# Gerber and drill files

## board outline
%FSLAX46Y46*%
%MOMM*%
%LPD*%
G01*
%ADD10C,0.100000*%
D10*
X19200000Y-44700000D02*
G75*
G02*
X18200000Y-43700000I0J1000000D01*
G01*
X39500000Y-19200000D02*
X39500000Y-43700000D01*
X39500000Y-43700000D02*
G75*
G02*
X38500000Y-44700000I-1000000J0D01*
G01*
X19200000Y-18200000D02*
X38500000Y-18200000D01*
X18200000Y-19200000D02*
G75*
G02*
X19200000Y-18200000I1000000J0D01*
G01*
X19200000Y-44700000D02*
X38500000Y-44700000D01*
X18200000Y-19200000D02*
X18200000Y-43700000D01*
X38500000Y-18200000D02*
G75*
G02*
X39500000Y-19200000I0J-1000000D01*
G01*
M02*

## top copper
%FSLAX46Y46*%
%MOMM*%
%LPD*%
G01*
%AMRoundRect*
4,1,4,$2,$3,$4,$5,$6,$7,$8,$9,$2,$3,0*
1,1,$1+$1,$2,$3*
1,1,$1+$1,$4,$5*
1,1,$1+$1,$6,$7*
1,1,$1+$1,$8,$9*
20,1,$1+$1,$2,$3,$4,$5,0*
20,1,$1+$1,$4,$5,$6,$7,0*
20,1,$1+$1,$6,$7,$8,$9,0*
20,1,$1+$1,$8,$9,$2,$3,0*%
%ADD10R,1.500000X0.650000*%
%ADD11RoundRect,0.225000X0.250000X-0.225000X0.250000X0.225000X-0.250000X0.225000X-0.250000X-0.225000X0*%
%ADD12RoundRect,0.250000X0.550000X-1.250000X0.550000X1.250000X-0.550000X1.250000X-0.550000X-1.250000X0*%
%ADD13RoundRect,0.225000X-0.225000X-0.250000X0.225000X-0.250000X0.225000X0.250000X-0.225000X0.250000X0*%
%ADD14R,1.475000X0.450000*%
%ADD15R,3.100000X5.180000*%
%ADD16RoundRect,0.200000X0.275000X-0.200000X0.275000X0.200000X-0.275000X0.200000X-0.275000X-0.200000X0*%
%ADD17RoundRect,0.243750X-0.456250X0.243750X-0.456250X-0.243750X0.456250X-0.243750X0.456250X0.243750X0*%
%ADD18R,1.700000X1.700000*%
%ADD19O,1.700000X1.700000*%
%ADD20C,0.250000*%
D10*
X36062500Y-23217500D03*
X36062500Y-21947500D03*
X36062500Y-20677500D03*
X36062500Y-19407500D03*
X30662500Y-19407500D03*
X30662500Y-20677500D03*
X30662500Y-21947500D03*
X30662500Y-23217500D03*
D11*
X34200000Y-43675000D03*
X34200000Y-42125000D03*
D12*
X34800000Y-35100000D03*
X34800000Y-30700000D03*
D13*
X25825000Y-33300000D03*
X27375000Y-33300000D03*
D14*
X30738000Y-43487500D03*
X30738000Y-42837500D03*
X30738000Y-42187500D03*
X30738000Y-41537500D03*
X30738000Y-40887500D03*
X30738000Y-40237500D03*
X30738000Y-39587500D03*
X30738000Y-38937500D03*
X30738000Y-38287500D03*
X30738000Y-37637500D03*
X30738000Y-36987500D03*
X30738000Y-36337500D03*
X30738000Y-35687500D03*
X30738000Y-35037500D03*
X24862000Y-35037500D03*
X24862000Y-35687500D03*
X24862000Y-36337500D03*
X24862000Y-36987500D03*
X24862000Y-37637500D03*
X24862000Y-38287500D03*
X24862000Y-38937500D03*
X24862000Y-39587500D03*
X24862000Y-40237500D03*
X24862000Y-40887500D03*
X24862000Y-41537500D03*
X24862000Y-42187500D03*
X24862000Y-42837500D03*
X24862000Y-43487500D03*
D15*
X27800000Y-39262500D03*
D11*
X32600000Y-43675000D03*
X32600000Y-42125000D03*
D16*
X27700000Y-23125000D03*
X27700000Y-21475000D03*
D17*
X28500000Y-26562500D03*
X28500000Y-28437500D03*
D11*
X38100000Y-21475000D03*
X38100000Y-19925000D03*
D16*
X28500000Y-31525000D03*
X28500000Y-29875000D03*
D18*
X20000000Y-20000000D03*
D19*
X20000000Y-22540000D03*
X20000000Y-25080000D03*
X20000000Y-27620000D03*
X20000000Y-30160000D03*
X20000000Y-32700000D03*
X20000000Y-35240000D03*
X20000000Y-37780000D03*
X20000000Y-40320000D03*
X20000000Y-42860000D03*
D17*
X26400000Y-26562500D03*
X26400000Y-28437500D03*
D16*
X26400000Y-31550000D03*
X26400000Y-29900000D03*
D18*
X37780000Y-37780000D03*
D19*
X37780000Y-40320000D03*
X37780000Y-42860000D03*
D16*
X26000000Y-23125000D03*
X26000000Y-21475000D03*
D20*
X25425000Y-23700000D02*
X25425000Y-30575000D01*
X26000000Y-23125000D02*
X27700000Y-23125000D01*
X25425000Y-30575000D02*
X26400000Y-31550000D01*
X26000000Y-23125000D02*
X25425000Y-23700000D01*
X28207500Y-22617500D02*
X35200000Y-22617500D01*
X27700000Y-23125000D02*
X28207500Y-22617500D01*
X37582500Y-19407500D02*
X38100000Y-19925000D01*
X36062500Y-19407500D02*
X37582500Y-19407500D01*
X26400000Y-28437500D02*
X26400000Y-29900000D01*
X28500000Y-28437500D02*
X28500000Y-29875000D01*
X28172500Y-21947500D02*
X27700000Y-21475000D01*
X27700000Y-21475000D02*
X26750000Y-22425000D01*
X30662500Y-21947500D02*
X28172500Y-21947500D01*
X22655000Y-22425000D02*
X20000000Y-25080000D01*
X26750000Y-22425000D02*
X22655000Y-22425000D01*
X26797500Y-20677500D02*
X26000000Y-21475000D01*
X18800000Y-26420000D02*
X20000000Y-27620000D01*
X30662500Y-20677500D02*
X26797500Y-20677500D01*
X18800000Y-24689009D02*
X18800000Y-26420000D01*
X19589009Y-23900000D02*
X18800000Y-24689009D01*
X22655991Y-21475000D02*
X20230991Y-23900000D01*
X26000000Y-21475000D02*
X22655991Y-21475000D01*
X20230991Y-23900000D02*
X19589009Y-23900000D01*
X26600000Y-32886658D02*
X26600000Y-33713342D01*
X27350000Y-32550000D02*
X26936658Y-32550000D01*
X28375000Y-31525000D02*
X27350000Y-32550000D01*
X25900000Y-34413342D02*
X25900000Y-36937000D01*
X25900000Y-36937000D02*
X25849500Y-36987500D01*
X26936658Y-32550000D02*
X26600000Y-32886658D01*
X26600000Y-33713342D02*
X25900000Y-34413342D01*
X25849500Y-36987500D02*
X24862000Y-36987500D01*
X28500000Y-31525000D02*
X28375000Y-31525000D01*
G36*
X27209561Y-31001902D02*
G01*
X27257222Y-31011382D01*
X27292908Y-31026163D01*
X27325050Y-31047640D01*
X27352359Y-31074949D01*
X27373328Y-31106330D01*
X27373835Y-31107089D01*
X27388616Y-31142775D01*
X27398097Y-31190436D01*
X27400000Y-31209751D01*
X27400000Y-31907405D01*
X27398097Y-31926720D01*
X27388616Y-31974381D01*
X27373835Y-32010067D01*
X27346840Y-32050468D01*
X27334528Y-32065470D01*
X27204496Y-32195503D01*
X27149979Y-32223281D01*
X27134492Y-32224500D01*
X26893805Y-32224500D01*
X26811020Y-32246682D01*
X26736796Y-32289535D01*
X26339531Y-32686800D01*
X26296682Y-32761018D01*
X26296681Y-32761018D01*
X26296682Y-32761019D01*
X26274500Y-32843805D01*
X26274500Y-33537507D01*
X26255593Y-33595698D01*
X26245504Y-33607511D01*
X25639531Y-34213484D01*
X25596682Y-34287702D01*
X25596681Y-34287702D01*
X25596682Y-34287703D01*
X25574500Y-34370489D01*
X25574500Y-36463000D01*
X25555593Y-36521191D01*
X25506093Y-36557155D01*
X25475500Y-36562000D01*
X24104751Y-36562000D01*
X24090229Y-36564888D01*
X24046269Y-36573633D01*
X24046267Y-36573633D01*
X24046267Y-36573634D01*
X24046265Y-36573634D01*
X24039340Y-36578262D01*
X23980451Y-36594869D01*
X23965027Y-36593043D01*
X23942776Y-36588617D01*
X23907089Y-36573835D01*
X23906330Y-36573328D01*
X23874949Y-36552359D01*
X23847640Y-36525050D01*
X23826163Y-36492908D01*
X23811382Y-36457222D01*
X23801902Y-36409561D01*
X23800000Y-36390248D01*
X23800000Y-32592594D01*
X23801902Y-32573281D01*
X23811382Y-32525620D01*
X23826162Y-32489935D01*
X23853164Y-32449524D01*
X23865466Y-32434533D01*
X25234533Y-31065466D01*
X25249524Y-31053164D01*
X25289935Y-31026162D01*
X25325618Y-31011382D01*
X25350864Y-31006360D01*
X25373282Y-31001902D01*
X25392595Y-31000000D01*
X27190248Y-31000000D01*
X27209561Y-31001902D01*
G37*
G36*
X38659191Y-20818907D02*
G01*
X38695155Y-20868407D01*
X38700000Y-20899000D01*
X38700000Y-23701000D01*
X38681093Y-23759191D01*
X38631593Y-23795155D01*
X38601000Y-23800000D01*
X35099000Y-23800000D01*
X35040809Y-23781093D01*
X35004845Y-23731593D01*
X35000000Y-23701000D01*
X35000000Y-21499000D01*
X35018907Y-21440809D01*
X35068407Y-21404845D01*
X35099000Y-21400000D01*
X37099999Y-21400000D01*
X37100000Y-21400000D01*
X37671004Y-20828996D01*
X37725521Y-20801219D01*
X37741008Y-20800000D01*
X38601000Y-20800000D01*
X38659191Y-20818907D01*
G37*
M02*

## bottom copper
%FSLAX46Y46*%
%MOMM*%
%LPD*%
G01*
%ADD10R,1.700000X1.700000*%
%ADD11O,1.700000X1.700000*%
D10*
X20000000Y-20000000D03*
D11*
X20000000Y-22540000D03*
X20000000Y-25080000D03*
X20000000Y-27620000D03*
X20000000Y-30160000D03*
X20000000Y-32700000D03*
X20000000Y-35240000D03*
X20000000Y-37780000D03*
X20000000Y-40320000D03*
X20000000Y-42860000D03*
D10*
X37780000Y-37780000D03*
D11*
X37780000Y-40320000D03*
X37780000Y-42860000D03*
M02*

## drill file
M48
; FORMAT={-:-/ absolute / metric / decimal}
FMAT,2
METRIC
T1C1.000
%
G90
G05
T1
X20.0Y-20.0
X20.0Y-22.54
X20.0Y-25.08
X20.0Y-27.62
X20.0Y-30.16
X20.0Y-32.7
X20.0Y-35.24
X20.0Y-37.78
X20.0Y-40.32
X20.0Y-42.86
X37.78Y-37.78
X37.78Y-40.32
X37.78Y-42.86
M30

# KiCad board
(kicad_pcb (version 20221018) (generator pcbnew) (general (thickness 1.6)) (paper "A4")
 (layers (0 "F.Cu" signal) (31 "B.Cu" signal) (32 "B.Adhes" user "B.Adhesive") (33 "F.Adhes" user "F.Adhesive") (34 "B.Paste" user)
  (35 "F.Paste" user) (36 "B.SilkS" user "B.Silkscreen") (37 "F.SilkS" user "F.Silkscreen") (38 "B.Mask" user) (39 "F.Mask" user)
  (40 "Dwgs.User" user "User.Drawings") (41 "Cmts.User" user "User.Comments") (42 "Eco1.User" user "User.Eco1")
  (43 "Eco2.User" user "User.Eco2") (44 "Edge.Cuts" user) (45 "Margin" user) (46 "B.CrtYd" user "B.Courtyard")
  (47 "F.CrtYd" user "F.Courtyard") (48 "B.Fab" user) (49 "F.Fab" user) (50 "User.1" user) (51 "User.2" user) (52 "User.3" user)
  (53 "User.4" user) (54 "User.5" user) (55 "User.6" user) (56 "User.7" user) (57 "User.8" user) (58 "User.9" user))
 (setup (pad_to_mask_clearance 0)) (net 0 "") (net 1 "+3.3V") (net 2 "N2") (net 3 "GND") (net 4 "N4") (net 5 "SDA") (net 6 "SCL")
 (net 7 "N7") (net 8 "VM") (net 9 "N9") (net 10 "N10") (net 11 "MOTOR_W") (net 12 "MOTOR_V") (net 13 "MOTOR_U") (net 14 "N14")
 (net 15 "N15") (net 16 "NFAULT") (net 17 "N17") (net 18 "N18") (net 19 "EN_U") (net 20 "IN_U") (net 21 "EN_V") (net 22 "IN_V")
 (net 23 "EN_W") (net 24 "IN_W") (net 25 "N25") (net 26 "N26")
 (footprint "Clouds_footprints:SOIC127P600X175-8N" (layer "F.Cu") (at 33.3625 21.3125 180)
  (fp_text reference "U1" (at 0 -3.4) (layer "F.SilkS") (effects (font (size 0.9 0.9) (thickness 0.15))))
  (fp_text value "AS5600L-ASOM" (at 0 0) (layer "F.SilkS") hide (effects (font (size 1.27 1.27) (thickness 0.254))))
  (pad "1" smd rect (at -2.7 -1.905 270) (size 0.65 1.5) (layers "F.Cu" "F.Paste" "F.Mask") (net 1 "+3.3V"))
  (pad "2" smd rect (at -2.7 -0.635 270) (size 0.65 1.5) (layers "F.Cu" "F.Paste" "F.Mask") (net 1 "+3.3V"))
  (pad "3" smd rect (at -2.7 0.635 270) (size 0.65 1.5) (layers "F.Cu" "F.Paste" "F.Mask") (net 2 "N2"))
  (pad "4" smd rect (at -2.7 1.905 270) (size 0.65 1.5) (layers "F.Cu" "F.Paste" "F.Mask") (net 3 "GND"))
  (pad "5" smd rect (at 2.7 1.905 270) (size 0.65 1.5) (layers "F.Cu" "F.Paste" "F.Mask") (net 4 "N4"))
  (pad "6" smd rect (at 2.7 0.635 270) (size 0.65 1.5) (layers "F.Cu" "F.Paste" "F.Mask") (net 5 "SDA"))
  (pad "7" smd rect (at 2.7 -0.635 270) (size 0.65 1.5) (layers "F.Cu" "F.Paste" "F.Mask") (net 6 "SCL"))
  (pad "8" smd rect (at 2.7 -1.905 270) (size 0.65 1.5) (layers "F.Cu" "F.Paste" "F.Mask") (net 3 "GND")))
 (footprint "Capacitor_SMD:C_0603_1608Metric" (layer "F.Cu") (at 34.2 42.9 90)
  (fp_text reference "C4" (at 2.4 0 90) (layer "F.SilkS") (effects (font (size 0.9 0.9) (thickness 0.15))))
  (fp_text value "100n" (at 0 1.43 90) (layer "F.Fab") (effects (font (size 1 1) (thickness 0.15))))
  (pad "1" smd roundrect (at -0.775 0 90) (size 0.9 0.95) (layers "F.Cu" "F.Paste" "F.Mask") (roundrect_rratio 0.25) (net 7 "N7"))
  (pad "2" smd roundrect (at 0.775 0 90) (size 0.9 0.95) (layers "F.Cu" "F.Paste" "F.Mask") (roundrect_rratio 0.25) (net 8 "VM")))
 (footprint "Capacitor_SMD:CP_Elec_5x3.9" (layer "F.Cu") (at 34.8 32.9 90)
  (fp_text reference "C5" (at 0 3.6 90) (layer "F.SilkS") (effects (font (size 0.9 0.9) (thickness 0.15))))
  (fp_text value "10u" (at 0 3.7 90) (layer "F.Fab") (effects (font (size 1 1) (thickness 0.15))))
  (pad "1" smd roundrect (at -2.2 0 90) (size 3 1.6) (layers "F.Cu" "F.Paste" "F.Mask") (roundrect_rratio 0.15625) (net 8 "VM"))
  (pad "2" smd roundrect (at 2.2 0 90) (size 3 1.6) (layers "F.Cu" "F.Paste" "F.Mask") (roundrect_rratio 0.15625) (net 3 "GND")))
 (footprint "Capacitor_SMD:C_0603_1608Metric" (layer "F.Cu") (at 26.6 33.3)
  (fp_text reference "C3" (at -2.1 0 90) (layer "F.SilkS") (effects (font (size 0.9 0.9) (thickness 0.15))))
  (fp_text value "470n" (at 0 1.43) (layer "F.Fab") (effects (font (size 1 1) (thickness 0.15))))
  (pad "1" smd roundrect (at -0.775 0) (size 0.9 0.95) (layers "F.Cu" "F.Paste" "F.Mask") (roundrect_rratio 0.25) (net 1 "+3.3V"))
  (pad "2" smd roundrect (at 0.775 0) (size 0.9 0.95) (layers "F.Cu" "F.Paste" "F.Mask") (roundrect_rratio 0.25) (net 3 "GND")))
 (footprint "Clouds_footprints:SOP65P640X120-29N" (layer "F.Cu") (at 27.8 39.2625 180)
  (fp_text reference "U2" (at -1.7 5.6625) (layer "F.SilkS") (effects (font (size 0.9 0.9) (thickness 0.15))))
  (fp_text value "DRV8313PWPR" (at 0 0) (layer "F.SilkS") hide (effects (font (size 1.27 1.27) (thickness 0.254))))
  (pad "1" smd rect (at -2.938 -4.225 270) (size 0.45 1.475) (layers "F.Cu" "F.Paste" "F.Mask") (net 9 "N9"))
  (pad "2" smd rect (at -2.938 -3.575 270) (size 0.45 1.475) (layers "F.Cu" "F.Paste" "F.Mask") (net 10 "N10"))
  (pad "3" smd rect (at -2.938 -2.925 270) (size 0.45 1.475) (layers "F.Cu" "F.Paste" "F.Mask") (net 7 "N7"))
  (pad "4" smd rect (at -2.938 -2.275 270) (size 0.45 1.475) (layers "F.Cu" "F.Paste" "F.Mask") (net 8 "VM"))
  (pad "5" smd rect (at -2.938 -1.625 270) (size 0.45 1.475) (layers "F.Cu" "F.Paste" "F.Mask") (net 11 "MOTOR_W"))
  (pad "6" smd rect (at -2.938 -0.975 270) (size 0.45 1.475) (layers "F.Cu" "F.Paste" "F.Mask") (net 3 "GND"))
  (pad "7" smd rect (at -2.938 -0.325 270) (size 0.45 1.475) (layers "F.Cu" "F.Paste" "F.Mask") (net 3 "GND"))
  (pad "8" smd rect (at -2.938 0.325 270) (size 0.45 1.475) (layers "F.Cu" "F.Paste" "F.Mask") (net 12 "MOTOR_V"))
  (pad "9" smd rect (at -2.938 0.975 270) (size 0.45 1.475) (layers "F.Cu" "F.Paste" "F.Mask") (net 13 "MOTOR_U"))
  (pad "10" smd rect (at -2.938 1.625 270) (size 0.45 1.475) (layers "F.Cu" "F.Paste" "F.Mask") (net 3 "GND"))
  (pad "11" smd rect (at -2.938 2.275 270) (size 0.45 1.475) (layers "F.Cu" "F.Paste" "F.Mask") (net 8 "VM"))
  (pad "12" smd rect (at -2.938 2.925 270) (size 0.45 1.475) (layers "F.Cu" "F.Paste" "F.Mask") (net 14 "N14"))
  (pad "13" smd rect (at -2.938 3.575 270) (size 0.45 1.475) (layers "F.Cu" "F.Paste" "F.Mask") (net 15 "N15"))
  (pad "14" smd rect (at -2.938 4.225 270) (size 0.45 1.475) (layers "F.Cu" "F.Paste" "F.Mask") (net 3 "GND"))
  (pad "15" smd rect (at 2.938 4.225 270) (size 0.45 1.475) (layers "F.Cu" "F.Paste" "F.Mask") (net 1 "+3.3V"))
  (pad "16" smd rect (at 2.938 3.575 270) (size 0.45 1.475) (layers "F.Cu" "F.Paste" "F.Mask") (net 1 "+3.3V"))
  (pad "17" smd rect (at 2.938 2.925 270) (size 0.45 1.475) (layers "F.Cu" "F.Paste" "F.Mask") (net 1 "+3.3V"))
  (pad "18" smd rect (at 2.938 2.275 270) (size 0.45 1.475) (layers "F.Cu" "F.Paste" "F.Mask") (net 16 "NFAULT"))
  (pad "19" smd rect (at 2.938 1.625 270) (size 0.45 1.475) (layers "F.Cu" "F.Paste" "F.Mask") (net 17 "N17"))
  (pad "20" smd rect (at 2.938 0.975 270) (size 0.45 1.475) (layers "F.Cu" "F.Paste" "F.Mask") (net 3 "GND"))
  (pad "21" smd rect (at 2.938 0.325 270) (size 0.45 1.475) (layers "F.Cu" "F.Paste" "F.Mask") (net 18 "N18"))
  (pad "22" smd rect (at 2.938 -0.325 270) (size 0.45 1.475) (layers "F.Cu" "F.Paste" "F.Mask") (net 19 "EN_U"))
  (pad "23" smd rect (at 2.938 -0.975 270) (size 0.45 1.475) (layers "F.Cu" "F.Paste" "F.Mask") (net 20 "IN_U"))
  (pad "24" smd rect (at 2.938 -1.625 270) (size 0.45 1.475) (layers "F.Cu" "F.Paste" "F.Mask") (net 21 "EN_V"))
  (pad "25" smd rect (at 2.938 -2.275 270) (size 0.45 1.475) (layers "F.Cu" "F.Paste" "F.Mask") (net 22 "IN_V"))
  (pad "26" smd rect (at 2.938 -2.925 270) (size 0.45 1.475) (layers "F.Cu" "F.Paste" "F.Mask") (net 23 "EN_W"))
  (pad "27" smd rect (at 2.938 -3.575 270) (size 0.45 1.475) (layers "F.Cu" "F.Paste" "F.Mask") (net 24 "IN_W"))
  (pad "28" smd rect (at 2.938 -4.225 270) (size 0.45 1.475) (layers "F.Cu" "F.Paste" "F.Mask") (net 3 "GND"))
  (pad "29" smd rect (at 0 0 180) (size 3.1 5.18) (layers "F.Cu" "F.Paste" "F.Mask") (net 3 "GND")))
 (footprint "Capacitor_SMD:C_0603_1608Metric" (layer "F.Cu") (at 32.6 42.9 90)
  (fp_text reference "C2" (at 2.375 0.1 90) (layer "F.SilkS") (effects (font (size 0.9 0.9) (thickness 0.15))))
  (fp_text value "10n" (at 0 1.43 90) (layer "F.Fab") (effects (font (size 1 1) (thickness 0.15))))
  (pad "1" smd roundrect (at -0.775 0 90) (size 0.9 0.95) (layers "F.Cu" "F.Paste" "F.Mask") (roundrect_rratio 0.25) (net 9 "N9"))
  (pad "2" smd roundrect (at 0.775 0 90) (size 0.9 0.95) (layers "F.Cu" "F.Paste" "F.Mask") (roundrect_rratio 0.25) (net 10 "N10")))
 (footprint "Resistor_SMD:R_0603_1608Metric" (layer "F.Cu") (at 27.7 22.3 90)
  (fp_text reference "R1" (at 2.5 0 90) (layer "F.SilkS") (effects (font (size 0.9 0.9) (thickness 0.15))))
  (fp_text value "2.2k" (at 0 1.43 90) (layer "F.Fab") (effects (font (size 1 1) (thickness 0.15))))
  (pad "1" smd roundrect (at -0.825 0 90) (size 0.8 0.95) (layers "F.Cu" "F.Paste" "F.Mask") (roundrect_rratio 0.25) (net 1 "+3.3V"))
  (pad "2" smd roundrect (at 0.825 0 90) (size 0.8 0.95) (layers "F.Cu" "F.Paste" "F.Mask") (roundrect_rratio 0.25) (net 6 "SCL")))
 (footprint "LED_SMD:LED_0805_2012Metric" (layer "F.Cu") (at 28.5 27.5 -90)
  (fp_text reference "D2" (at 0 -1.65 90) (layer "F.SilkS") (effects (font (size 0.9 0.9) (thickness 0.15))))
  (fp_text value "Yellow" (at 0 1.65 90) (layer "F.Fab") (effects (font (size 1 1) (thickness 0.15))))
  (pad "1" smd roundrect (at -0.9375 0 270) (size 0.975 1.4) (layers "F.Cu" "F.Paste" "F.Mask") (roundrect_rratio 0.25) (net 3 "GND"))
  (pad "2" smd roundrect (at 0.9375 0 270) (size 0.975 1.4) (layers "F.Cu" "F.Paste" "F.Mask") (roundrect_rratio 0.25) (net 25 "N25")))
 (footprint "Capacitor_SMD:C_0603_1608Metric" (layer "F.Cu") (at 38.1 20.7 90)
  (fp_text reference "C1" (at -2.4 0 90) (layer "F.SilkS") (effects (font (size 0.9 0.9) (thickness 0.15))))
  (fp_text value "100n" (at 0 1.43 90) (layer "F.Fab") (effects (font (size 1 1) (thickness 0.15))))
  (pad "1" smd roundrect (at -0.775 0 90) (size 0.9 0.95) (layers "F.Cu" "F.Paste" "F.Mask") (roundrect_rratio 0.25) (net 1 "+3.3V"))
  (pad "2" smd roundrect (at 0.775 0 90) (size 0.9 0.95) (layers "F.Cu" "F.Paste" "F.Mask") (roundrect_rratio 0.25) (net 3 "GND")))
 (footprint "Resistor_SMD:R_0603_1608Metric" (layer "F.Cu") (at 28.5 30.7 90)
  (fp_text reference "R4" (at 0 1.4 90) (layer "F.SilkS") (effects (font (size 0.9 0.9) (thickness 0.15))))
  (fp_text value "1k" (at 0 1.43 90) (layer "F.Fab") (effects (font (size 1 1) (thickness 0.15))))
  (pad "1" smd roundrect (at -0.825 0 90) (size 0.8 0.95) (layers "F.Cu" "F.Paste" "F.Mask") (roundrect_rratio 0.25) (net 16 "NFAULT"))
  (pad "2" smd roundrect (at 0.825 0 90) (size 0.8 0.95) (layers "F.Cu" "F.Paste" "F.Mask") (roundrect_rratio 0.25) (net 25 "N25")))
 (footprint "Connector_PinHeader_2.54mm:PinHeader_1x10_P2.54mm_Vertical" (layer "F.Cu") (at 20 20)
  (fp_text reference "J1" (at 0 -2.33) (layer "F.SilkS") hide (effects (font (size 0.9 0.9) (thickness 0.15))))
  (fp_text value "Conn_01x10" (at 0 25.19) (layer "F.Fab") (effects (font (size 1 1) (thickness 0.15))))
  (pad "1" thru_hole rect (at 0 0) (size 1.7 1.7) (drill 1) (layers "*.Cu" "*.Mask") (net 8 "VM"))
  (pad "2" thru_hole oval (at 0 2.54) (size 1.7 1.7) (drill 1) (layers "*.Cu" "*.Mask") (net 3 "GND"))
  (pad "3" thru_hole oval (at 0 5.08) (size 1.7 1.7) (drill 1) (layers "*.Cu" "*.Mask") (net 6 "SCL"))
  (pad "4" thru_hole oval (at 0 7.62) (size 1.7 1.7) (drill 1) (layers "*.Cu" "*.Mask") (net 5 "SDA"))
  (pad "5" thru_hole oval (at 0 10.16) (size 1.7 1.7) (drill 1) (layers "*.Cu" "*.Mask") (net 19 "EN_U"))
  (pad "6" thru_hole oval (at 0 12.7) (size 1.7 1.7) (drill 1) (layers "*.Cu" "*.Mask") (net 20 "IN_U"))
  (pad "7" thru_hole oval (at 0 15.24) (size 1.7 1.7) (drill 1) (layers "*.Cu" "*.Mask") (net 21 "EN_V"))
  (pad "8" thru_hole oval (at 0 17.78) (size 1.7 1.7) (drill 1) (layers "*.Cu" "*.Mask") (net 22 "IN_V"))
  (pad "9" thru_hole oval (at 0 20.32) (size 1.7 1.7) (drill 1) (layers "*.Cu" "*.Mask") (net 23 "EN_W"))
  (pad "10" thru_hole oval (at 0 22.86) (size 1.7 1.7) (drill 1) (layers "*.Cu" "*.Mask") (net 24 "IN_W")))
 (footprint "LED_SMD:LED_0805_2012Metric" (layer "F.Cu") (at 26.4 27.5 -90)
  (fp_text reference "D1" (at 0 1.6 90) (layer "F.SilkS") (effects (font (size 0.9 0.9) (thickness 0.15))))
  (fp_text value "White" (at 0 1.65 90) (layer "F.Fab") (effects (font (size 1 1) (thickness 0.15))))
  (pad "1" smd roundrect (at -0.9375 0 270) (size 0.975 1.4) (layers "F.Cu" "F.Paste" "F.Mask") (roundrect_rratio 0.25) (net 3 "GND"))
  (pad "2" smd roundrect (at 0.9375 0 270) (size 0.975 1.4) (layers "F.Cu" "F.Paste" "F.Mask") (roundrect_rratio 0.25) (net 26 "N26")))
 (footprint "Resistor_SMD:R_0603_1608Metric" (layer "F.Cu") (at 26.4 30.725 90)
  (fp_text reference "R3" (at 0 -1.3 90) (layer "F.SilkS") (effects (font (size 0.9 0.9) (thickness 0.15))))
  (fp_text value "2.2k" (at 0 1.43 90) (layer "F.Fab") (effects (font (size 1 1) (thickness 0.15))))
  (pad "1" smd roundrect (at -0.825 0 90) (size 0.8 0.95) (layers "F.Cu" "F.Paste" "F.Mask") (roundrect_rratio 0.25) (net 1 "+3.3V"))
  (pad "2" smd roundrect (at 0.825 0 90) (size 0.8 0.95) (layers "F.Cu" "F.Paste" "F.Mask") (roundrect_rratio 0.25) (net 26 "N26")))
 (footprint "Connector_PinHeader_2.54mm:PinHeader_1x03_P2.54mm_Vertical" (layer "F.Cu") (at 37.78 37.78)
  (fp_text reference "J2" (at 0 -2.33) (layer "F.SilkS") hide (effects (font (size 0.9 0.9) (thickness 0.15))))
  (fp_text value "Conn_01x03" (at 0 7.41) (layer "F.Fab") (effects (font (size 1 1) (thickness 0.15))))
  (pad "1" thru_hole rect (at 0 0) (size 1.7 1.7) (drill 1) (layers "*.Cu" "*.Mask") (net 13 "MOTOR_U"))
  (pad "2" thru_hole oval (at 0 2.54) (size 1.7 1.7) (drill 1) (layers "*.Cu" "*.Mask") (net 12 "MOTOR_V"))
  (pad "3" thru_hole oval (at 0 5.08) (size 1.7 1.7) (drill 1) (layers "*.Cu" "*.Mask") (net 11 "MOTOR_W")))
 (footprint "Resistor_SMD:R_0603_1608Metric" (layer "F.Cu") (at 26 22.3 90)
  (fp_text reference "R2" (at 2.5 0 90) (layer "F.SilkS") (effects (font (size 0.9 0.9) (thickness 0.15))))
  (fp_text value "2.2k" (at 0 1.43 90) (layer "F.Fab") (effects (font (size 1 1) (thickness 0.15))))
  (pad "1" smd roundrect (at -0.825 0 90) (size 0.8 0.95) (layers "F.Cu" "F.Paste" "F.Mask") (roundrect_rratio 0.25) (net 1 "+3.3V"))
  (pad "2" smd roundrect (at 0.825 0 90) (size 0.8 0.95) (layers "F.Cu" "F.Paste" "F.Mask") (roundrect_rratio 0.25) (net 5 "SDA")))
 (gr_arc (start 19.2 44.7) (mid 18.492894 44.407106) (end 18.2 43.7) (stroke (width 0.1) (type default)) (layer "Edge.Cuts"))
 (gr_line (start 39.5 19.2) (end 39.5 43.7) (stroke (width 0.1) (type default)) (layer "Edge.Cuts"))
 (gr_arc (start 39.5 43.7) (mid 39.207107 44.407106) (end 38.5 44.7) (stroke (width 0.1) (type default)) (layer "Edge.Cuts"))
 (gr_line (start 19.2 18.2) (end 38.5 18.2) (stroke (width 0.1) (type default)) (layer "Edge.Cuts"))
 (gr_arc (start 18.2 19.2) (mid 18.492893 18.492894) (end 19.2 18.2) (stroke (width 0.1) (type default)) (layer "Edge.Cuts"))
 (gr_line (start 19.2 44.7) (end 38.5 44.7) (stroke (width 0.1) (type default)) (layer "Edge.Cuts"))
 (gr_line (start 18.2 19.2) (end 18.2 43.7) (stroke (width 0.1) (type default)) (layer "Edge.Cuts"))
 (gr_arc (start 38.5 18.2) (mid 39.207106 18.492894) (end 39.5 19.2) (stroke (width 0.1) (type default)) (layer "Edge.Cuts"))
 (segment (start 25.425 23.7) (end 25.425 30.575) (width 0.25) (layer "F.Cu") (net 1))
 (segment (start 26 23.125) (end 27.7 23.125) (width 0.25) (layer "F.Cu") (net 1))
 (segment (start 25.425 30.575) (end 26.4 31.55) (width 0.25) (layer "F.Cu") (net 1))
 (segment (start 26 23.125) (end 25.425 23.7) (width 0.25) (layer "F.Cu") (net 1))
 (segment (start 28.2075 22.6175) (end 35.2 22.6175) (width 0.25) (layer "F.Cu") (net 1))
 (segment (start 27.7 23.125) (end 28.2075 22.6175) (width 0.25) (layer "F.Cu") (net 1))
 (segment (start 37.5825 19.4075) (end 38.1 19.925) (width 0.25) (layer "F.Cu") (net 3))
 (segment (start 36.0625 19.4075) (end 37.5825 19.4075) (width 0.25) (layer "F.Cu") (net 3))
 (segment (start 26.4 28.4375) (end 26.4 29.9) (width 0.25) (layer "F.Cu") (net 26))
 (segment (start 28.5 28.4375) (end 28.5 29.875) (width 0.25) (layer "F.Cu") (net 25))
 (segment (start 28.1725 21.9475) (end 27.7 21.475) (width 0.25) (layer "F.Cu") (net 6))
 (segment (start 27.7 21.475) (end 26.75 22.425) (width 0.25) (layer "F.Cu") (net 6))
 (segment (start 30.6625 21.9475) (end 28.1725 21.9475) (width 0.25) (layer "F.Cu") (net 6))
 (segment (start 22.655 22.425) (end 20 25.08) (width 0.25) (layer "F.Cu") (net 6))
 (segment (start 26.75 22.425) (end 22.655 22.425) (width 0.25) (layer "F.Cu") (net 6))
 (segment (start 26.7975 20.6775) (end 26 21.475) (width 0.25) (layer "F.Cu") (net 5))
 (segment (start 18.8 26.42) (end 20 27.62) (width 0.25) (layer "F.Cu") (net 5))
 (segment (start 30.6625 20.6775) (end 26.7975 20.6775) (width 0.25) (layer "F.Cu") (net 5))
 (segment (start 18.8 24.689009) (end 18.8 26.42) (width 0.25) (layer "F.Cu") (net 5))
 (segment (start 19.589009 23.9) (end 18.8 24.689009) (width 0.25) (layer "F.Cu") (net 5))
 (segment (start 22.655991 21.475) (end 20.230991 23.9) (width 0.25) (layer "F.Cu") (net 5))
 (segment (start 26 21.475) (end 22.655991 21.475) (width 0.25) (layer "F.Cu") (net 5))
 (segment (start 20.230991 23.9) (end 19.589009 23.9) (width 0.25) (layer "F.Cu") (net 5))
 (segment (start 26.6 32.886658) (end 26.6 33.713342) (width 0.25) (layer "F.Cu") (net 16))
 (segment (start 27.35 32.55) (end 26.936658 32.55) (width 0.25) (layer "F.Cu") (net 16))
 (segment (start 28.375 31.525) (end 27.35 32.55) (width 0.25) (layer "F.Cu") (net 16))
 (segment (start 25.9 34.413342) (end 25.9 36.937) (width 0.25) (layer "F.Cu") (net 16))
 (segment (start 25.9 36.937) (end 25.8495 36.9875) (width 0.25) (layer "F.Cu") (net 16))
 (segment (start 26.936658 32.55) (end 26.6 32.886658) (width 0.25) (layer "F.Cu") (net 16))
 (segment (start 26.6 33.713342) (end 25.9 34.413342) (width 0.25) (layer "F.Cu") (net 16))
 (segment (start 25.8495 36.9875) (end 24.862 36.9875) (width 0.25) (layer "F.Cu") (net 16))
 (segment (start 28.5 31.525) (end 28.375 31.525) (width 0.25) (layer "F.Cu") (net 16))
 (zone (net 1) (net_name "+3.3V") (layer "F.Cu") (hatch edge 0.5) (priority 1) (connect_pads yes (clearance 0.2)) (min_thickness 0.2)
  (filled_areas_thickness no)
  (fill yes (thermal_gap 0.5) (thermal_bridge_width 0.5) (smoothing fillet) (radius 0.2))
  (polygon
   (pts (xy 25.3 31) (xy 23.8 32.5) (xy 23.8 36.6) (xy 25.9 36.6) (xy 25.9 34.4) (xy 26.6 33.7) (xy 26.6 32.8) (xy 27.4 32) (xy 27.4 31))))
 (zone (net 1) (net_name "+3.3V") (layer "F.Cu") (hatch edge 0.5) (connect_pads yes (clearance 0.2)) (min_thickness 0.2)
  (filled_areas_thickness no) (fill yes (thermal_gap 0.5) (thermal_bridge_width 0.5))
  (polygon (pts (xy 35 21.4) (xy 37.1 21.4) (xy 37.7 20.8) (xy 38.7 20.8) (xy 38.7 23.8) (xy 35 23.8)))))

